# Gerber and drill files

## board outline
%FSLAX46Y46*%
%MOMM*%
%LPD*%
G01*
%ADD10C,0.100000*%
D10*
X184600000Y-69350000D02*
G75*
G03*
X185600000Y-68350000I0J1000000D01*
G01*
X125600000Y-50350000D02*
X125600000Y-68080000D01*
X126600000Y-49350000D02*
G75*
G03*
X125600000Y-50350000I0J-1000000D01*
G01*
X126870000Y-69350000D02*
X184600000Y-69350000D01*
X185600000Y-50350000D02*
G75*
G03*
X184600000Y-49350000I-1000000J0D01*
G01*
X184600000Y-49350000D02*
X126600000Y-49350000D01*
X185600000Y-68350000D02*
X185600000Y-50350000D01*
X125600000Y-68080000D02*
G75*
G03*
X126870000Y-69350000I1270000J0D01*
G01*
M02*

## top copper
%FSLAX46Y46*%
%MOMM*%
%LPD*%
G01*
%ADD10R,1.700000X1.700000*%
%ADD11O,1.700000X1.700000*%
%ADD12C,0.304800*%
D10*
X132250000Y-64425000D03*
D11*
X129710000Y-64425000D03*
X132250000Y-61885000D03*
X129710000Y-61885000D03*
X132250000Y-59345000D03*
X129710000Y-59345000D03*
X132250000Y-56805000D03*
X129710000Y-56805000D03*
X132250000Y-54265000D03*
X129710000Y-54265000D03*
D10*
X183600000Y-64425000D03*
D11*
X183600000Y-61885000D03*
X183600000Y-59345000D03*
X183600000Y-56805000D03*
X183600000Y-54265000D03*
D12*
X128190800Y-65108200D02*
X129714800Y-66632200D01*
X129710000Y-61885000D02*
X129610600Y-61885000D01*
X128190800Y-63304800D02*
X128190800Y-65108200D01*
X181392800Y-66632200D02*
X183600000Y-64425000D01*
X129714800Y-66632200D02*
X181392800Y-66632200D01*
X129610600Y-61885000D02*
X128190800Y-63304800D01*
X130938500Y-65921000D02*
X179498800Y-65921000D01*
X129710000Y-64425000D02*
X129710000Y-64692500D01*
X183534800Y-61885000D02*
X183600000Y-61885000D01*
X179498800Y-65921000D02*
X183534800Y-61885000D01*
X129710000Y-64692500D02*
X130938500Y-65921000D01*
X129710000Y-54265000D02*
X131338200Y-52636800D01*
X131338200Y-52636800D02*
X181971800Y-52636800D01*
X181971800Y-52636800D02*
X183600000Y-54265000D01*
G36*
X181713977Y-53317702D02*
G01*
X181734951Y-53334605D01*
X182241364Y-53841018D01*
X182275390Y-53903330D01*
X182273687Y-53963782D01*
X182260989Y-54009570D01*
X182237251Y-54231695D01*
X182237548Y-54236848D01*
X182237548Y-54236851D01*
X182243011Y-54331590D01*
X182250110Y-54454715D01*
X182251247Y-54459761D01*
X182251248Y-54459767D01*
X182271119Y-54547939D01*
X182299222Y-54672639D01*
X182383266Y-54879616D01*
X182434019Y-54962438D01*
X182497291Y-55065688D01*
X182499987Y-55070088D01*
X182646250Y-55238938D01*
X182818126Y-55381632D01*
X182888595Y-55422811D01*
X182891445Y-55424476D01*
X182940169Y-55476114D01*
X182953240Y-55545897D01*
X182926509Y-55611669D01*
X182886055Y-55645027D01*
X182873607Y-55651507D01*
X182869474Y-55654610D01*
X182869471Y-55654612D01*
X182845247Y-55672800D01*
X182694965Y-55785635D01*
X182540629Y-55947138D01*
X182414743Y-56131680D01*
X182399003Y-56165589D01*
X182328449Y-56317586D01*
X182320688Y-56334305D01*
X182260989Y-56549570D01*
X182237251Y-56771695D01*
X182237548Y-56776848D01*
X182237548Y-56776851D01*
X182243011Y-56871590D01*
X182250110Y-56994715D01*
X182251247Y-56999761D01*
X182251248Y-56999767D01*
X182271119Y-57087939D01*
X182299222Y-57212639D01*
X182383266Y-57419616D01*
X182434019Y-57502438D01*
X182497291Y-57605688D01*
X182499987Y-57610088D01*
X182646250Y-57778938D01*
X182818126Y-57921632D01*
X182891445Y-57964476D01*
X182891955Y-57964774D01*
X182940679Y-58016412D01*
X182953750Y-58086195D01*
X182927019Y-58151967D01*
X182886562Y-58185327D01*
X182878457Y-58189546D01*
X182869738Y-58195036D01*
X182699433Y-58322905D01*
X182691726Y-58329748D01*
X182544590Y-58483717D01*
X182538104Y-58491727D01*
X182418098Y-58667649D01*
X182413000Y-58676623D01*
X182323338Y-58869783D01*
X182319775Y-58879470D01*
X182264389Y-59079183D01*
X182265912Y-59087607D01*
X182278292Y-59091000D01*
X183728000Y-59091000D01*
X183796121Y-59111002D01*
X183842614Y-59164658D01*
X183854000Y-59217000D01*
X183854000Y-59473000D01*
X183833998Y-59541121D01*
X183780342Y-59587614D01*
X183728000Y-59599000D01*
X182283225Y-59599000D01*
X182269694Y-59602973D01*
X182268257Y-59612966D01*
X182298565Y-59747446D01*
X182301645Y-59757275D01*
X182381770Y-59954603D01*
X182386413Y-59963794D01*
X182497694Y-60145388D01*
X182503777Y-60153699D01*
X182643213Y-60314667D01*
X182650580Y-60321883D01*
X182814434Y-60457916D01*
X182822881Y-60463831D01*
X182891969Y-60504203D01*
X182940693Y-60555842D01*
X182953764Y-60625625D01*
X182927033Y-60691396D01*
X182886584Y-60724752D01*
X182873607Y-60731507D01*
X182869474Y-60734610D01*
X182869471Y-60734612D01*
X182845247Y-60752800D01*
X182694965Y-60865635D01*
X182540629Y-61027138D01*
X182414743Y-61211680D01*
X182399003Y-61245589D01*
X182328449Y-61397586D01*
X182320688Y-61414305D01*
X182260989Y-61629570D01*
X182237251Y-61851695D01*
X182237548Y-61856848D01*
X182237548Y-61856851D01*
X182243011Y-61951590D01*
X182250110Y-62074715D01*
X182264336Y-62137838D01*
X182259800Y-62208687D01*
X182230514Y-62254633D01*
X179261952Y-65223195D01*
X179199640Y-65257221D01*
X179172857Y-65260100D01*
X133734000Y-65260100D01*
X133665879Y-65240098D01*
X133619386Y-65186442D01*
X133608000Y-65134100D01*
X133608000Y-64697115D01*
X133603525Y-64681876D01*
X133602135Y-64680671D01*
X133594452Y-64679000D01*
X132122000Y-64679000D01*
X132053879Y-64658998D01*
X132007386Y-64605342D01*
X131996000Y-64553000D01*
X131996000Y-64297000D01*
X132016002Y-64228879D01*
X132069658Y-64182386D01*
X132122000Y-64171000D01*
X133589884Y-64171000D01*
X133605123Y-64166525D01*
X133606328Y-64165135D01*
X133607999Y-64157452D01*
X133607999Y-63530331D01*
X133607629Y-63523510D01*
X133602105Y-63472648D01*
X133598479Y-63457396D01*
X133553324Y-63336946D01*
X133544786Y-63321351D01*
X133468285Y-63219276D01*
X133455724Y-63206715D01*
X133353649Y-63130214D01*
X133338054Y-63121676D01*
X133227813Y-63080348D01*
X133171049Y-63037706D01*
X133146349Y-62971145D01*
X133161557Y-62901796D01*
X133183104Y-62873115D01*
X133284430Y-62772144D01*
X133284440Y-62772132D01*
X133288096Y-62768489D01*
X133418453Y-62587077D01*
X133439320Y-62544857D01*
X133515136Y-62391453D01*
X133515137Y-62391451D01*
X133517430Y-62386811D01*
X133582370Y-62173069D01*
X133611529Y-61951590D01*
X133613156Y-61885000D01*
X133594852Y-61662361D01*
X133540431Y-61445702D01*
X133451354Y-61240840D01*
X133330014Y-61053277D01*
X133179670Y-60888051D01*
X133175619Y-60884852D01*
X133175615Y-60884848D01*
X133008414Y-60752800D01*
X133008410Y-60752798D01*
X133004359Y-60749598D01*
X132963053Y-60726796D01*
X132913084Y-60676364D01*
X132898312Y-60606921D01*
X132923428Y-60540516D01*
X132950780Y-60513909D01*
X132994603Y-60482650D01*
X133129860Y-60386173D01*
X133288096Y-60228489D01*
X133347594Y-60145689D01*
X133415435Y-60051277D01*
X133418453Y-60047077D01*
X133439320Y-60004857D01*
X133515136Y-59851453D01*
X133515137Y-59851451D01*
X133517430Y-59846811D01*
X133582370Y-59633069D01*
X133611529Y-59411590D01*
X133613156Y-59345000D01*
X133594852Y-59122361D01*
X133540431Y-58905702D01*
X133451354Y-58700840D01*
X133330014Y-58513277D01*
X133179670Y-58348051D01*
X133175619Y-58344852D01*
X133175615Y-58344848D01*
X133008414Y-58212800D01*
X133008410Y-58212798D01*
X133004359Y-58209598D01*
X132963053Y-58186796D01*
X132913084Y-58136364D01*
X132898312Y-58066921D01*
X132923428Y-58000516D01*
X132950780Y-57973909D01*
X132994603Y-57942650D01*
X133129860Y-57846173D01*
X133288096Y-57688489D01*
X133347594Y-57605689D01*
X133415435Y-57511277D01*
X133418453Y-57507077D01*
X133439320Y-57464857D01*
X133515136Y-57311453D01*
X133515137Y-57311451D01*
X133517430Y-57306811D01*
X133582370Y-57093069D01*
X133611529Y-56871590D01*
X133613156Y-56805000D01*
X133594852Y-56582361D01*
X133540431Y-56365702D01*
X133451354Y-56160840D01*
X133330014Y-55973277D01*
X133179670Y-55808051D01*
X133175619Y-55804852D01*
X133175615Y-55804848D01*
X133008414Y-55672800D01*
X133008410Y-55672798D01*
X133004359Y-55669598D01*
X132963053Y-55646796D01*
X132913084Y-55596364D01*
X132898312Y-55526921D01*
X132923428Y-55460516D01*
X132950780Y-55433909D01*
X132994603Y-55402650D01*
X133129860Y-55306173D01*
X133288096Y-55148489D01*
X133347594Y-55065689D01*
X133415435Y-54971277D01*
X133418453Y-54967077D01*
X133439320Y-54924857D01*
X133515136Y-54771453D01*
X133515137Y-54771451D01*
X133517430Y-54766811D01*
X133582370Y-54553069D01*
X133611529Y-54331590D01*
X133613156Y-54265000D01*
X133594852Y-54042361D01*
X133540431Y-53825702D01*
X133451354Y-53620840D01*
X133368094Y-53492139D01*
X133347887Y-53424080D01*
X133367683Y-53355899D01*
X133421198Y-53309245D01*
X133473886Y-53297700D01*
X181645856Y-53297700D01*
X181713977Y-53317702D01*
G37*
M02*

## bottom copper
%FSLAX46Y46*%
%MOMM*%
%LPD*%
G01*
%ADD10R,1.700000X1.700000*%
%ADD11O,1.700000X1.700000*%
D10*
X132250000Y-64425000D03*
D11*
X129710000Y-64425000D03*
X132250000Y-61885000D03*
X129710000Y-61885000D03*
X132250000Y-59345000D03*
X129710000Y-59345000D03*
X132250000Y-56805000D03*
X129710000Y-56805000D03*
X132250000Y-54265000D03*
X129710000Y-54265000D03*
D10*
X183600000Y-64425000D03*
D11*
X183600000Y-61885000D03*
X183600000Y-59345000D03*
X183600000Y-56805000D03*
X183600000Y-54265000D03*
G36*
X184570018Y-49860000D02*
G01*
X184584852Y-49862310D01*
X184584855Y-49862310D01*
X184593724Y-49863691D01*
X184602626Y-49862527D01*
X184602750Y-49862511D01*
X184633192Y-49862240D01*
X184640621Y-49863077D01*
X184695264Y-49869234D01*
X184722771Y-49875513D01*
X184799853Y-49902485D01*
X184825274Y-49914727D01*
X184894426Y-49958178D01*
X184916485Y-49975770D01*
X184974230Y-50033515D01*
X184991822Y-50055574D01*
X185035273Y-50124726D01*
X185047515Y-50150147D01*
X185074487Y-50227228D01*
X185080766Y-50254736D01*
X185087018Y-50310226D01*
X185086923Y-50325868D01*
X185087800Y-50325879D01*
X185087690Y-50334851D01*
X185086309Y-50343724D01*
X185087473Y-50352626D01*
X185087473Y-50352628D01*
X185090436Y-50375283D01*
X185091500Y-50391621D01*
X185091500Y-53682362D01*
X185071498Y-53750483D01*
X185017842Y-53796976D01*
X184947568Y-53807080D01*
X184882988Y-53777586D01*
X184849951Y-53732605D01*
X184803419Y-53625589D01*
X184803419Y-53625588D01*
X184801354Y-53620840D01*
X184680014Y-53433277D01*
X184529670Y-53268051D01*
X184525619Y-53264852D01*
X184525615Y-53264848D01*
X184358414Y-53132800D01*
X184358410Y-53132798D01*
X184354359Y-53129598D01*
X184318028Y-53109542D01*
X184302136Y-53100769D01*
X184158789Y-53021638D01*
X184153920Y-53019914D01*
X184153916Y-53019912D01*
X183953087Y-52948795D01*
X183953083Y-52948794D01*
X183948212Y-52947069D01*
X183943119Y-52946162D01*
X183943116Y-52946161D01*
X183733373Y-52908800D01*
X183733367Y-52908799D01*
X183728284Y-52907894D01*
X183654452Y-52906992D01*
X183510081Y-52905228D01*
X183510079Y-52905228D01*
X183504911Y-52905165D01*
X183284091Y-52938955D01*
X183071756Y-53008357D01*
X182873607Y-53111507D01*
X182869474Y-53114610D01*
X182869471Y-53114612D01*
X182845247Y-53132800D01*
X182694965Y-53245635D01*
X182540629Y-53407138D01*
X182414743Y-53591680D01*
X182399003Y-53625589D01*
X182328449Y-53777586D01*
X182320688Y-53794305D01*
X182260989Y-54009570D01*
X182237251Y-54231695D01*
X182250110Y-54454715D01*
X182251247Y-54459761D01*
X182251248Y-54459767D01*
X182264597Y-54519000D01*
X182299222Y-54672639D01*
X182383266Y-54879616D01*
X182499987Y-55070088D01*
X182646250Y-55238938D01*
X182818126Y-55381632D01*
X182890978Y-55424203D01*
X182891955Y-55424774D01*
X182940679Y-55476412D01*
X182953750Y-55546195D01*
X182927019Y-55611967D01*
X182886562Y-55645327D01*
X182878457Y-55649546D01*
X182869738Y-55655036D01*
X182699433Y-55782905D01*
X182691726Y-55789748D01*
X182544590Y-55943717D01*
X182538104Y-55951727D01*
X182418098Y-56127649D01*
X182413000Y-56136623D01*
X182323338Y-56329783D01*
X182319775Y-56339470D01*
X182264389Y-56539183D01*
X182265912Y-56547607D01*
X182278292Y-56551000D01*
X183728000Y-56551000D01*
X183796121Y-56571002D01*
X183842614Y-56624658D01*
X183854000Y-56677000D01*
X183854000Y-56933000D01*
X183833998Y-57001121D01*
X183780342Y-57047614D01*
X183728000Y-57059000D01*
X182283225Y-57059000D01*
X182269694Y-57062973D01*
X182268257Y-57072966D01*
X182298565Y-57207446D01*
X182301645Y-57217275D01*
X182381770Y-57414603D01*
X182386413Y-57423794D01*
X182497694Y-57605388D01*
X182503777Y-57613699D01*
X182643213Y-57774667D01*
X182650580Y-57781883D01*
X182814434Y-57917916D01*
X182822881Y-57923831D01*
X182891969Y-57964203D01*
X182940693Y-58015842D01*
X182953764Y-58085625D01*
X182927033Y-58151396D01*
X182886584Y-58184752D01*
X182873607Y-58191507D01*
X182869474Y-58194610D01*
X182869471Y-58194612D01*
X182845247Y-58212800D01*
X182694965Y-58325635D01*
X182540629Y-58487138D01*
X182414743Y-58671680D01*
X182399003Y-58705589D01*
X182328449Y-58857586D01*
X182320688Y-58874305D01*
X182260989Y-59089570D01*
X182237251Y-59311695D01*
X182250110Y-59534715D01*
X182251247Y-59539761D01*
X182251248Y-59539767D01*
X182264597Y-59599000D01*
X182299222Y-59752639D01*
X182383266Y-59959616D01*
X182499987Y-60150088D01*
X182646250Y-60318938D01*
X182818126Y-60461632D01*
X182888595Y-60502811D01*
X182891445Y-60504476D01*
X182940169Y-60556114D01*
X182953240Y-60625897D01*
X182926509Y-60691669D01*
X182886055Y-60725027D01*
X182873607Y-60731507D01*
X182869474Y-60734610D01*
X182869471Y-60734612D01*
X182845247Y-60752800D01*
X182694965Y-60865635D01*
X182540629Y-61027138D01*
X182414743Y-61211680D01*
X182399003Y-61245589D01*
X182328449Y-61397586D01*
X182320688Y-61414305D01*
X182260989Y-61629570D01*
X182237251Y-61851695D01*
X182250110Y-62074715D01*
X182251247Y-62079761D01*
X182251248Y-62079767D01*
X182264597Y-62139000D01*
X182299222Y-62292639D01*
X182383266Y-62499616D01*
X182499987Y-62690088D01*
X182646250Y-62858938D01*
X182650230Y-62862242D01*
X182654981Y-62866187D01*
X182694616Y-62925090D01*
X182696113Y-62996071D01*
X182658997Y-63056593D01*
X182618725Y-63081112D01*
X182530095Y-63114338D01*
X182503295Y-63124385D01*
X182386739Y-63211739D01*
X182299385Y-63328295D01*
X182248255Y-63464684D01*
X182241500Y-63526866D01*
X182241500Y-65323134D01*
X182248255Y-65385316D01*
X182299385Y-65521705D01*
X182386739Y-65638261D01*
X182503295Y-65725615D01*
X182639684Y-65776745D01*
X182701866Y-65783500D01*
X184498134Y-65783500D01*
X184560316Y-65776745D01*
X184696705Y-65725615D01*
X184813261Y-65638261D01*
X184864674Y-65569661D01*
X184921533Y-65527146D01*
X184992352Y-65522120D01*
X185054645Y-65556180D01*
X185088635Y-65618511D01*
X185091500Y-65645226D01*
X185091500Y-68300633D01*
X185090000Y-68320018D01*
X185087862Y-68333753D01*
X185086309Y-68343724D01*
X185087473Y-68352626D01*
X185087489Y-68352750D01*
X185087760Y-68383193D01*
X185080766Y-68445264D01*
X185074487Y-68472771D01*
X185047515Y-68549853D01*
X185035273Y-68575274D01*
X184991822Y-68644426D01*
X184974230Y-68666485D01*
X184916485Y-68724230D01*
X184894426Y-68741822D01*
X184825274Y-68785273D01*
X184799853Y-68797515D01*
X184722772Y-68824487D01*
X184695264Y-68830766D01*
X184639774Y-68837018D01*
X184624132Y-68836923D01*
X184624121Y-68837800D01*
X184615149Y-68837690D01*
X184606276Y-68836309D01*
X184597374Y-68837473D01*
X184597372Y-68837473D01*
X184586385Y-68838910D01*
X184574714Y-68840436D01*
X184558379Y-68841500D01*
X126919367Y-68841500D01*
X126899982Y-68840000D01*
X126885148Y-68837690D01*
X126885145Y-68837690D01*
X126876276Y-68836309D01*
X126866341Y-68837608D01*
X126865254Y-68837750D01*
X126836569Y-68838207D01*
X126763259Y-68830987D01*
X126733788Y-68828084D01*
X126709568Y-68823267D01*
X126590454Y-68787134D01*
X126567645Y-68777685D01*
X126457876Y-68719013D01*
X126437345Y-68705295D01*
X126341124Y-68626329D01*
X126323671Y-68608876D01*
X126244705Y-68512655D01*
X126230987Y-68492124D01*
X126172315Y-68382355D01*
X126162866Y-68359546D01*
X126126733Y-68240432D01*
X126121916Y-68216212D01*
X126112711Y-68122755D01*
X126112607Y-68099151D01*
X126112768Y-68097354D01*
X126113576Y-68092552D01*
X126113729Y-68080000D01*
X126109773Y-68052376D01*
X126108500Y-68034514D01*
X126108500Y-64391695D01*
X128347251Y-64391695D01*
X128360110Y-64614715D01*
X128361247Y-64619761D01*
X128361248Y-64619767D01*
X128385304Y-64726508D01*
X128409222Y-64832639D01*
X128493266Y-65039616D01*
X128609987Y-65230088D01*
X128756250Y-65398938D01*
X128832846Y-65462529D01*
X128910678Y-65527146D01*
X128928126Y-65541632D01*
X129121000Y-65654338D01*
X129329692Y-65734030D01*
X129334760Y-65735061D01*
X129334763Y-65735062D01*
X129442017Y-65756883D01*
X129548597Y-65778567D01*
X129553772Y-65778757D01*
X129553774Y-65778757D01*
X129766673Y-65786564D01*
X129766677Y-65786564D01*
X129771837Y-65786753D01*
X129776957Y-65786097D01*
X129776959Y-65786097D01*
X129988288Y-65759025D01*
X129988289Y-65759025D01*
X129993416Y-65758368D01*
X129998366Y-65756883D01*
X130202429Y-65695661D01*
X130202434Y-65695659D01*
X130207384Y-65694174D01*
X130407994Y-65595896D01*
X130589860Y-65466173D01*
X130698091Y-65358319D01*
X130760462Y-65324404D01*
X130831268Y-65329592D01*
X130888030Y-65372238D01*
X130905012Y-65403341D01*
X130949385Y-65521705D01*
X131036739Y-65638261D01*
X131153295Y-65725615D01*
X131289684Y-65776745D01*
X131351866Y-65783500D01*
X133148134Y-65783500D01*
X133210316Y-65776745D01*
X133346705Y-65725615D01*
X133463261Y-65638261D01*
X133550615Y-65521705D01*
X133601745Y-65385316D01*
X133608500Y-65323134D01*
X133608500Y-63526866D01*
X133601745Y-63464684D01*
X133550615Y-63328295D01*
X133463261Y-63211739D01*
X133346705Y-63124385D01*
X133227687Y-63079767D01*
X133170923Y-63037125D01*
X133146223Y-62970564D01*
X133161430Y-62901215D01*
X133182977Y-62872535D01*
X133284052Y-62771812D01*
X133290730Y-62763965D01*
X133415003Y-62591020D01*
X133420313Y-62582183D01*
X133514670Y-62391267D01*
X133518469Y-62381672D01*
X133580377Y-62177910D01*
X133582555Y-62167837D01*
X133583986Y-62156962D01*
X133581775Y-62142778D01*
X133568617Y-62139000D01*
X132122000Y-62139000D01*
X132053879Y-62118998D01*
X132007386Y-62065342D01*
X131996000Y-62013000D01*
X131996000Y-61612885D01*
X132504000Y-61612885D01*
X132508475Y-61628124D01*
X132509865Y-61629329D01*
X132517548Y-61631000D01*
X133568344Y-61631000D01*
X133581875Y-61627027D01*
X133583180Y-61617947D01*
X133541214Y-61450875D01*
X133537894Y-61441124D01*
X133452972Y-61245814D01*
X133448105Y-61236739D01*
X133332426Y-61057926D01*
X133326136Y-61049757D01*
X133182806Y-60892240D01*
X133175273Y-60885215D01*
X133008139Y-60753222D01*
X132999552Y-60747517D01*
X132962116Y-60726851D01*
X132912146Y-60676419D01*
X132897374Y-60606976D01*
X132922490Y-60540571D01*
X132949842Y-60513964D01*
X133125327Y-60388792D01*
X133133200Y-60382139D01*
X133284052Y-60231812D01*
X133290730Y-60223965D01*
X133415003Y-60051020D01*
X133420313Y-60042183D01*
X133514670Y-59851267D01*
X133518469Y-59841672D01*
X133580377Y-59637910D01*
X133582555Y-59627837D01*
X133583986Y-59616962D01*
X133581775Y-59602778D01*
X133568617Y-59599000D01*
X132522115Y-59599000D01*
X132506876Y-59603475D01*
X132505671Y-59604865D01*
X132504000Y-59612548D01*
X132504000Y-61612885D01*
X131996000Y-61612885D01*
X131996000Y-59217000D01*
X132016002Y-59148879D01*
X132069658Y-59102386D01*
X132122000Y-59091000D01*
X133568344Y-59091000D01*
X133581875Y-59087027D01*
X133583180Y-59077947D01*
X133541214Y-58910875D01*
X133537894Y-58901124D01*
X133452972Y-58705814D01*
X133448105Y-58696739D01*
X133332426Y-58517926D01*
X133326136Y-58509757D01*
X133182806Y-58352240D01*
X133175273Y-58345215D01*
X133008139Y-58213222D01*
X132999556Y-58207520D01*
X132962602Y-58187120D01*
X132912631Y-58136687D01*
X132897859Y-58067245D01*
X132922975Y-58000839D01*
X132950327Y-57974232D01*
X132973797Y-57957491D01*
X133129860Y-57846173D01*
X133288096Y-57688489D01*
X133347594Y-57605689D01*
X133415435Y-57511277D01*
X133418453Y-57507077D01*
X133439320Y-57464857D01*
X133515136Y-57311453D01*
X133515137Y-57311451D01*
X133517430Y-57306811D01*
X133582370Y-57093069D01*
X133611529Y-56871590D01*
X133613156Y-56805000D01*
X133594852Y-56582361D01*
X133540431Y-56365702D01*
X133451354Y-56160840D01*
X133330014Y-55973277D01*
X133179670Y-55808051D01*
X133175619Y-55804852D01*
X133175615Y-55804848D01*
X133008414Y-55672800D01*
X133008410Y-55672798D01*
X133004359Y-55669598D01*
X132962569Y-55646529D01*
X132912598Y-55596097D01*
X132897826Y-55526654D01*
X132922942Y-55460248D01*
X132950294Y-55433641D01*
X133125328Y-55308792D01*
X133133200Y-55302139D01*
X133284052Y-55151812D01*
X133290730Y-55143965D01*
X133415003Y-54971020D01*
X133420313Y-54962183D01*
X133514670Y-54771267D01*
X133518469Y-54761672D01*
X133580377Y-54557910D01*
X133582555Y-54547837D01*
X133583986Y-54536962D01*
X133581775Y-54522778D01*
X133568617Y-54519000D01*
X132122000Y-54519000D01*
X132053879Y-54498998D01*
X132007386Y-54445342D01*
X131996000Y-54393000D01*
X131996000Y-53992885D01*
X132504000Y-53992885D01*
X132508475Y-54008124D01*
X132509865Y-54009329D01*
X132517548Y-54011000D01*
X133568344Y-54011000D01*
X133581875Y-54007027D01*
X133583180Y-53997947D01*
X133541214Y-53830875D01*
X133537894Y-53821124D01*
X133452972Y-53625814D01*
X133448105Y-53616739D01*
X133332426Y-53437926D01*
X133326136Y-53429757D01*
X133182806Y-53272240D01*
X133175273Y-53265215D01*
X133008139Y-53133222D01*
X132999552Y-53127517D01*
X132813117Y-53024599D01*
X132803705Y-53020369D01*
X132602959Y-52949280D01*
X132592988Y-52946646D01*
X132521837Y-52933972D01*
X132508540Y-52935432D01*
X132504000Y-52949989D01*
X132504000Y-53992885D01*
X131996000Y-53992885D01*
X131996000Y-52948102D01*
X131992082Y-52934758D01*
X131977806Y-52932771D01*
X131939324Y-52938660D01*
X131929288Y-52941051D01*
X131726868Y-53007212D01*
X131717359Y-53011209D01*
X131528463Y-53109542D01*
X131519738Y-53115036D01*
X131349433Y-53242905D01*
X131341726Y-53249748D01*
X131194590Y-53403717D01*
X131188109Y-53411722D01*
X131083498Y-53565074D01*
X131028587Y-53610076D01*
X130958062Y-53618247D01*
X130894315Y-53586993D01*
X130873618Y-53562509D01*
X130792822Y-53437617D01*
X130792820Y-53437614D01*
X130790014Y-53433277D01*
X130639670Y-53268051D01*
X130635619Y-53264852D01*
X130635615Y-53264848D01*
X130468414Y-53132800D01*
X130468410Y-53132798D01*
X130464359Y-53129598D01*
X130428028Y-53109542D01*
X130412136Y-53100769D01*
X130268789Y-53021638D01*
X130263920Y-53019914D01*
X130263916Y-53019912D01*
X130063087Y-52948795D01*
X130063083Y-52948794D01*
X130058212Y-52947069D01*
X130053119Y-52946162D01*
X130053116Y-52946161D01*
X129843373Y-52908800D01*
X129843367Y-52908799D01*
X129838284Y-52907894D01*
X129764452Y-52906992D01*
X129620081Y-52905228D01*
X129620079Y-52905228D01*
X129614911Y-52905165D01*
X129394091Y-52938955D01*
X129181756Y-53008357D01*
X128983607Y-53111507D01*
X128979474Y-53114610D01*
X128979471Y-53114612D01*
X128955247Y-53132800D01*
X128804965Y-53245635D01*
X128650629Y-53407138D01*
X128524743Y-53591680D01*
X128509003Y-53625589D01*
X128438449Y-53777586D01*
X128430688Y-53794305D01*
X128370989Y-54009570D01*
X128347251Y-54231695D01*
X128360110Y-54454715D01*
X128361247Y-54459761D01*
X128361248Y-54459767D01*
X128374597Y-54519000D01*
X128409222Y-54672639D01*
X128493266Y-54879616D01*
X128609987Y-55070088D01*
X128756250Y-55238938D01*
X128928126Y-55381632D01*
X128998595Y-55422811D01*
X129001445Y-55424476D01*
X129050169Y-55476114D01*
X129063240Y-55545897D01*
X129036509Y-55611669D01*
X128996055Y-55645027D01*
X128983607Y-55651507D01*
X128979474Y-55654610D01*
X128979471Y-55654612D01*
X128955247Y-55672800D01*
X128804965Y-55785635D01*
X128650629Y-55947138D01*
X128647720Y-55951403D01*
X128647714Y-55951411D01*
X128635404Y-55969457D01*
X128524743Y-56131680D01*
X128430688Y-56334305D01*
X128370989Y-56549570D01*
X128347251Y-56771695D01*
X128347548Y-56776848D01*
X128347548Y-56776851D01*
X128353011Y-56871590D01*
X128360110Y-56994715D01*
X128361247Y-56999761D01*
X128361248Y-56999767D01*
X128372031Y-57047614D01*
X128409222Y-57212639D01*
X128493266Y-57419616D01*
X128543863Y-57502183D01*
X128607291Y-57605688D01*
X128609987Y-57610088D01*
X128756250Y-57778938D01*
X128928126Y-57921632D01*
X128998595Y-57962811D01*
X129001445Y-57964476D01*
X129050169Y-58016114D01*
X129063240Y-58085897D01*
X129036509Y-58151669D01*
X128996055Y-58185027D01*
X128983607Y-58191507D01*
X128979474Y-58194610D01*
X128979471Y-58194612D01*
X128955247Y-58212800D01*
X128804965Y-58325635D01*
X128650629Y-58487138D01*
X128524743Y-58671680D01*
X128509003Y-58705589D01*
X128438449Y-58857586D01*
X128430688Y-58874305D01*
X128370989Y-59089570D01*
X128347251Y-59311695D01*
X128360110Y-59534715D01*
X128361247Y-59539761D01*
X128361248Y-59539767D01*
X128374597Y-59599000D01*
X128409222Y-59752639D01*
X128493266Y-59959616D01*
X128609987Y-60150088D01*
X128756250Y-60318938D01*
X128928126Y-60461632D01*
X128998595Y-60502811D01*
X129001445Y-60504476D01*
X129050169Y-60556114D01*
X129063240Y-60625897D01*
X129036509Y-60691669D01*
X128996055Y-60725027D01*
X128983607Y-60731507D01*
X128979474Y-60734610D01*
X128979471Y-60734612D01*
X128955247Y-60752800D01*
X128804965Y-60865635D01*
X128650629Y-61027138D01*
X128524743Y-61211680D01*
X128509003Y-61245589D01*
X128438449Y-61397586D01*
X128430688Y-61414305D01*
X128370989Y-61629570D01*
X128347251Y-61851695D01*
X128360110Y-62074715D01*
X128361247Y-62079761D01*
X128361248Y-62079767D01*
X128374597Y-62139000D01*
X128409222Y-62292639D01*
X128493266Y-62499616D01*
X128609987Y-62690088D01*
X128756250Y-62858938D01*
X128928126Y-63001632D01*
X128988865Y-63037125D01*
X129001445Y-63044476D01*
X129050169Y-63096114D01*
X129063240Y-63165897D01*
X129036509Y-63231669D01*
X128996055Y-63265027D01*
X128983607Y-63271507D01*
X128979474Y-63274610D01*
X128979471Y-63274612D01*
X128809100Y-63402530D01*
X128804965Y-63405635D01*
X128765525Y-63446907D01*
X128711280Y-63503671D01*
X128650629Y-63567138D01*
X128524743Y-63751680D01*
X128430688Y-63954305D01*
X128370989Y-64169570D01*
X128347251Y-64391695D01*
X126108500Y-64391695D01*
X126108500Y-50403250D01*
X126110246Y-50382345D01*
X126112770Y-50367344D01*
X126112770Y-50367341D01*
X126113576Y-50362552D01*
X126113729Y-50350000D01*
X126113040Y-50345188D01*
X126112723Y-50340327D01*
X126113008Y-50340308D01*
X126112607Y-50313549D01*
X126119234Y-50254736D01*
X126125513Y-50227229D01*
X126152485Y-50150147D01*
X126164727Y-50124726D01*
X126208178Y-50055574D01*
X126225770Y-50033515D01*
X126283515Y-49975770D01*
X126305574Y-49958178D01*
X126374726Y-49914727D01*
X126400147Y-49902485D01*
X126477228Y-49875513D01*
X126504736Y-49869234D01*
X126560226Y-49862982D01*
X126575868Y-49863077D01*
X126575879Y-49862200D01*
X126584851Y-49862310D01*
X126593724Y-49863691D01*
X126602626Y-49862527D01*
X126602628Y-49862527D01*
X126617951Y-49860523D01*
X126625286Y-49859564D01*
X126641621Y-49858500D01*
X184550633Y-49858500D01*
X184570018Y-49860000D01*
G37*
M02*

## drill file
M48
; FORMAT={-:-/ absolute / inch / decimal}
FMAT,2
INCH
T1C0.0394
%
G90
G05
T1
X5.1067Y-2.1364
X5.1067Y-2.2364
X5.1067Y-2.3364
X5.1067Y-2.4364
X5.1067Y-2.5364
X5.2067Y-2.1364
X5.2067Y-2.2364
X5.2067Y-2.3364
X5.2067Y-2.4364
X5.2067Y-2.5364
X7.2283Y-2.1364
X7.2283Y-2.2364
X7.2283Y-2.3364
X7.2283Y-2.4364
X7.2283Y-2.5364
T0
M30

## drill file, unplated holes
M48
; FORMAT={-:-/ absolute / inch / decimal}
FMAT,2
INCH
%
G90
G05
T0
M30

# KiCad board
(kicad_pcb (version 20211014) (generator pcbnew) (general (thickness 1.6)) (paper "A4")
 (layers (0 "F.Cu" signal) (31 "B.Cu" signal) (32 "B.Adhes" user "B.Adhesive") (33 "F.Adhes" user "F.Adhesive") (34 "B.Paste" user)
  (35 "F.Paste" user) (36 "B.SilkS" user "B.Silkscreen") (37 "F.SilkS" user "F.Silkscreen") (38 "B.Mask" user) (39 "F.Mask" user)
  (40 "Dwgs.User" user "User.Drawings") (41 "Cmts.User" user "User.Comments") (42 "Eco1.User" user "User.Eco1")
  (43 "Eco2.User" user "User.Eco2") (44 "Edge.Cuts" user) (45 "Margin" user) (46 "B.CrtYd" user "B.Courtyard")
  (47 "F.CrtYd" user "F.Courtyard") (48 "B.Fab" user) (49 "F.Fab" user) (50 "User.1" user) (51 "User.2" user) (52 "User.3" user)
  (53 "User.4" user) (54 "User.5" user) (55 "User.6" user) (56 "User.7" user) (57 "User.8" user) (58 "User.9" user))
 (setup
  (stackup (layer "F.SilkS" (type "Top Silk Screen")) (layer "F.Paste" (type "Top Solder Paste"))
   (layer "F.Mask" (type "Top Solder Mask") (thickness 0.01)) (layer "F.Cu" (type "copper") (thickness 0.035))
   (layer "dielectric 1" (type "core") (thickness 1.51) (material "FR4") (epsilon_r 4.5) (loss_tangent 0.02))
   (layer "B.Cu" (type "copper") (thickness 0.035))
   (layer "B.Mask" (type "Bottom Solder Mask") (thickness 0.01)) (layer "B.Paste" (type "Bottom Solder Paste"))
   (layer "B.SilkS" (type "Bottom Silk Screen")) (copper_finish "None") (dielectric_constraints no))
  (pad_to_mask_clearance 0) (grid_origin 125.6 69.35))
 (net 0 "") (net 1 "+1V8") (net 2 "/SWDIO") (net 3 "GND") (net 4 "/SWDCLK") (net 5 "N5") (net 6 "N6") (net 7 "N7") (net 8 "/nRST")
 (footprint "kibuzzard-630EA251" (layer "F.Cu") (at 142.057657 59.35)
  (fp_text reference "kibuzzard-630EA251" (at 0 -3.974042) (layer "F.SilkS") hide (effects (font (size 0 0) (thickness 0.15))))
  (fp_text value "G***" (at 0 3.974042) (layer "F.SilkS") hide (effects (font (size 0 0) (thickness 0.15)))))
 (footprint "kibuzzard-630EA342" (layer "F.Cu") (at 141.607601 56.81)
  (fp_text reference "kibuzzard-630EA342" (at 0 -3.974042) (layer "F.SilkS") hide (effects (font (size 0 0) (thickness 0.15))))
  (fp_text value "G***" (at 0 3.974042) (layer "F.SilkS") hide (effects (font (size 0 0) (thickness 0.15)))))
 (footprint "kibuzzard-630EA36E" (layer "F.Cu") (at 138.142882 61.89)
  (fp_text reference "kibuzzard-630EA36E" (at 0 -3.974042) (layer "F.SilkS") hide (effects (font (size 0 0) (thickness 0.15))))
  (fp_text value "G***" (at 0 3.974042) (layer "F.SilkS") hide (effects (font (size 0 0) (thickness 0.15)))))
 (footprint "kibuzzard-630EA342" (layer "F.Cu") (at 138.585 59.35)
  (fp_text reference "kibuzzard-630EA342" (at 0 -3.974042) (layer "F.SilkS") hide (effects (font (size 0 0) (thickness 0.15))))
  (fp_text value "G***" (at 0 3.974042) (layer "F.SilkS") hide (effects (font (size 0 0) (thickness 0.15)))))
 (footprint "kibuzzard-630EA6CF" (layer "F.Cu") (at 178.028025 54.27)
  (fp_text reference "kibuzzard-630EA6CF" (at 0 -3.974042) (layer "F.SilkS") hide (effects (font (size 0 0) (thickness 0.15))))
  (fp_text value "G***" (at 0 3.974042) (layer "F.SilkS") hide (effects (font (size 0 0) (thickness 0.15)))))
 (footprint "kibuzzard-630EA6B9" (layer "F.Cu") (at 173.785573 51.493604)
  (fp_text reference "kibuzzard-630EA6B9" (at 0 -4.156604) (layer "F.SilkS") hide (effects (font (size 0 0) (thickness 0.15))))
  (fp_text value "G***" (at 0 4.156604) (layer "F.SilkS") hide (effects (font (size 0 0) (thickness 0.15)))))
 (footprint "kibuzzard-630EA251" (layer "F.Cu") (at 142.057657 54.27)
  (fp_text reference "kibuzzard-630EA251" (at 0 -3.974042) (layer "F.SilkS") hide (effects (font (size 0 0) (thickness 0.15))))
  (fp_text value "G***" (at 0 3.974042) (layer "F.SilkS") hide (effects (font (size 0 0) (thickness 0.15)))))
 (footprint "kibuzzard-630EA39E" (layer "F.Cu") (at 144.828496 51.311042)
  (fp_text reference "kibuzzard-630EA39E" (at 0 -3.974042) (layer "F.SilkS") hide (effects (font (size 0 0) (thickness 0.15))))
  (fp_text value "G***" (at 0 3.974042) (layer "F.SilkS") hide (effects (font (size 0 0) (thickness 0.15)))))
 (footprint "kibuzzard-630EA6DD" (layer "F.Cu") (at 179.185312 56.81)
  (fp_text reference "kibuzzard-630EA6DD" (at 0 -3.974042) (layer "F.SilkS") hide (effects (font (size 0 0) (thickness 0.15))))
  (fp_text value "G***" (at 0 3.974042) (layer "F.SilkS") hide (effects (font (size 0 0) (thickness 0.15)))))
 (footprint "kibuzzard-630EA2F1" (layer "F.Cu") (at 136.977657 54.27)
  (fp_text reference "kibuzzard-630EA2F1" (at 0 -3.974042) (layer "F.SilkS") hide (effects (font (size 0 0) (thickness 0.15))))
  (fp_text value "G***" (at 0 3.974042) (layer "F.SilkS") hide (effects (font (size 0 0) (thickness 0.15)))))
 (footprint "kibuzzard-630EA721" (layer "F.Cu") (at 179.200393 61.89)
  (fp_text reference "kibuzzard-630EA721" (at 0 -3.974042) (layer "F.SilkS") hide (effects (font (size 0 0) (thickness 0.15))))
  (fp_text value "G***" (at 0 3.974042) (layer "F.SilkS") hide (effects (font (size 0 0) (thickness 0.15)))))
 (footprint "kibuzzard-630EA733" (layer "F.Cu") (at 179.19325 64.43)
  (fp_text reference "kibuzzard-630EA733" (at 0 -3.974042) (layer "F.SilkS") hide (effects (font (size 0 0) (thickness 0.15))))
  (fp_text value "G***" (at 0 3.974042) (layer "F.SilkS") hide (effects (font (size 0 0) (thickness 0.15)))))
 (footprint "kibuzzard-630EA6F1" (layer "F.Cu") (at 179.225 59.35)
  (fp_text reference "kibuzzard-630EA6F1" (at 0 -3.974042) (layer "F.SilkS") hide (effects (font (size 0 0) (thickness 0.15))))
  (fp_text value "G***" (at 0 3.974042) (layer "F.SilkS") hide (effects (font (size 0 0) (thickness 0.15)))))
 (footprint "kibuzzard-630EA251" (layer "F.Cu") (at 142.057657 61.89)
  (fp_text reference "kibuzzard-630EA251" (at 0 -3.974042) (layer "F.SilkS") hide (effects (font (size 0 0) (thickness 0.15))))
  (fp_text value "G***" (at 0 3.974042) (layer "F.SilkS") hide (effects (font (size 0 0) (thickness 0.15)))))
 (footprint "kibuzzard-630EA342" (layer "F.Cu") (at 138.585 56.81)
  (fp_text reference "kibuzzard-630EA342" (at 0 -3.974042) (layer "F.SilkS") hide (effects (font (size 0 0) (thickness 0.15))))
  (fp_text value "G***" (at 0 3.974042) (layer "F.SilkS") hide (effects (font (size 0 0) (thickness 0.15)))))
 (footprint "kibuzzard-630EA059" (layer "F.Cu") (at 142.017969 64.43)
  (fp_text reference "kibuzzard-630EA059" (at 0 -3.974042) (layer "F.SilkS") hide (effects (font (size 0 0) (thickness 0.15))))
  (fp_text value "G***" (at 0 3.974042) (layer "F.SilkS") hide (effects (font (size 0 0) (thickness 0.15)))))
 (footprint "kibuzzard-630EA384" (layer "F.Cu") (at 138.150025 64.43)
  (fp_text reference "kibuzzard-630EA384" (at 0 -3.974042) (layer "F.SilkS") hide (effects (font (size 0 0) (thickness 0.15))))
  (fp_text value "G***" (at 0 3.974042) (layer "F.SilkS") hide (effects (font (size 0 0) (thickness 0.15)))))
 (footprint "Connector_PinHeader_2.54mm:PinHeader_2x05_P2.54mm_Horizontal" (layer "F.Cu") (at 132.25 64.425 180)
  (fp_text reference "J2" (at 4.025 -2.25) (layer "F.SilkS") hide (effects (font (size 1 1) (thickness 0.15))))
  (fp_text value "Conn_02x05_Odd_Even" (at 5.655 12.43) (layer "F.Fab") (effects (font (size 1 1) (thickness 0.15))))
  (pad "1" thru_hole rect (at 0 0 180) (size 1.7 1.7) (drill 1) (layers *.Cu *.Mask) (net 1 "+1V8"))
  (pad "2" thru_hole oval (at 2.54 0 180) (size 1.7 1.7) (drill 1) (layers *.Cu *.Mask) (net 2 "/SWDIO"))
  (pad "3" thru_hole oval (at 0 2.54 180) (size 1.7 1.7) (drill 1) (layers *.Cu *.Mask) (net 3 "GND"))
  (pad "4" thru_hole oval (at 2.54 2.54 180) (size 1.7 1.7) (drill 1) (layers *.Cu *.Mask) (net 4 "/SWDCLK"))
  (pad "5" thru_hole oval (at 0 5.08 180) (size 1.7 1.7) (drill 1) (layers *.Cu *.Mask) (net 3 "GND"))
  (pad "6" thru_hole oval (at 2.54 5.08 180) (size 1.7 1.7) (drill 1) (layers *.Cu *.Mask) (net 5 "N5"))
  (pad "7" thru_hole oval (at 0 7.62 180) (size 1.7 1.7) (drill 1) (layers *.Cu *.Mask) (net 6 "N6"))
  (pad "8" thru_hole oval (at 2.54 7.62 180) (size 1.7 1.7) (drill 1) (layers *.Cu *.Mask) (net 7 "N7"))
  (pad "9" thru_hole oval (at 0 10.16 180) (size 1.7 1.7) (drill 1) (layers *.Cu *.Mask) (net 3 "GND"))
  (pad "10" thru_hole oval (at 2.54 10.16 180) (size 1.7 1.7) (drill 1) (layers *.Cu *.Mask) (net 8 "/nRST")))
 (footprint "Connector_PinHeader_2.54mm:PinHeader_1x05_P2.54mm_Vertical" (layer "B.Cu") (at 183.6 64.425)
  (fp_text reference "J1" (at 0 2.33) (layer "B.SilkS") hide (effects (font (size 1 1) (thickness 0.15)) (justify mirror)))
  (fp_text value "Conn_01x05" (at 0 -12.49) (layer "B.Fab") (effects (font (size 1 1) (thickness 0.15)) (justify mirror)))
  (pad "1" thru_hole rect (at 0 0) (size 1.7 1.7) (drill 1) (layers *.Cu *.Mask) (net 4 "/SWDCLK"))
  (pad "2" thru_hole oval (at 0 -2.54) (size 1.7 1.7) (drill 1) (layers *.Cu *.Mask) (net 2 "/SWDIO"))
  (pad "3" thru_hole oval (at 0 -5.08) (size 1.7 1.7) (drill 1) (layers *.Cu *.Mask) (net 1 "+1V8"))
  (pad "4" thru_hole oval (at 0 -7.62) (size 1.7 1.7) (drill 1) (layers *.Cu *.Mask) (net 3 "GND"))
  (pad "5" thru_hole oval (at 0 -10.16) (size 1.7 1.7) (drill 1) (layers *.Cu *.Mask) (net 8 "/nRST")))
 (gr_arc (start 185.6 68.35) (mid 185.307107 69.057107) (end 184.6 69.35) (layer "Edge.Cuts") (width 0.1))
 (gr_line (start 125.6 50.35) (end 125.6 68.08) (layer "Edge.Cuts") (width 0.1))
 (gr_arc (start 125.6 50.35) (mid 125.892893 49.642893) (end 126.6 49.35) (layer "Edge.Cuts") (width 0.1))
 (gr_line (start 126.87 69.35) (end 184.6 69.35) (layer "Edge.Cuts") (width 0.1))
 (gr_arc (start 184.6 49.35) (mid 185.307107 49.642893) (end 185.6 50.35) (layer "Edge.Cuts") (width 0.1))
 (gr_line (start 184.6 49.35) (end 126.6 49.35) (layer "Edge.Cuts") (width 0.1))
 (gr_line (start 185.6 68.35) (end 185.6 50.35) (layer "Edge.Cuts") (width 0.1))
 (gr_arc (start 126.87 69.35) (mid 125.971974 68.978026) (end 125.6 68.08) (layer "Edge.Cuts") (width 0.1))
 (segment (start 128.1908 65.1082) (end 129.7148 66.6322) (width 0.3048) (layer "F.Cu") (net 4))
 (segment (start 129.71 61.885) (end 129.6106 61.885) (width 0.3048) (layer "F.Cu") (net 4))
 (segment (start 128.1908 63.3048) (end 128.1908 65.1082) (width 0.3048) (layer "F.Cu") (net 4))
 (segment (start 181.3928 66.6322) (end 183.6 64.425) (width 0.3048) (layer "F.Cu") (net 4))
 (segment (start 129.7148 66.6322) (end 181.3928 66.6322) (width 0.3048) (layer "F.Cu") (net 4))
 (segment (start 129.6106 61.885) (end 128.1908 63.3048) (width 0.3048) (layer "F.Cu") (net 4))
 (segment (start 130.9385 65.921) (end 179.4988 65.921) (width 0.3048) (layer "F.Cu") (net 2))
 (segment (start 129.71 64.425) (end 129.71 64.6925) (width 0.3048) (layer "F.Cu") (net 2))
 (segment (start 183.5348 61.885) (end 183.6 61.885) (width 0.3048) (layer "F.Cu") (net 2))
 (segment (start 179.4988 65.921) (end 183.5348 61.885) (width 0.3048) (layer "F.Cu") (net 2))
 (segment (start 129.71 64.6925) (end 130.9385 65.921) (width 0.3048) (layer "F.Cu") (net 2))
 (segment (start 129.71 54.265) (end 131.3382 52.6368) (width 0.3048) (layer "F.Cu") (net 8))
 (segment (start 131.3382 52.6368) (end 181.9718 52.6368) (width 0.3048) (layer "F.Cu") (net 8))
 (segment (start 181.9718 52.6368) (end 183.6 54.265) (width 0.3048) (layer "F.Cu") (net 8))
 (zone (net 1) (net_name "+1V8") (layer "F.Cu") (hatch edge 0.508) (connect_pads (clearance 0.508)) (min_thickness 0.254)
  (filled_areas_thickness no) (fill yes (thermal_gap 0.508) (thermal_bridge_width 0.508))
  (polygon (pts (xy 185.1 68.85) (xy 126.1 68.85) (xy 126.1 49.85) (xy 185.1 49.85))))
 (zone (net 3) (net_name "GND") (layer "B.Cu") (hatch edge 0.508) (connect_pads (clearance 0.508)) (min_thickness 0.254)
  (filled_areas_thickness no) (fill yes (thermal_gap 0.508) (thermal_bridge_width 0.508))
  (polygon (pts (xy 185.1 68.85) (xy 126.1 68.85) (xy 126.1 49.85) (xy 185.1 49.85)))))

